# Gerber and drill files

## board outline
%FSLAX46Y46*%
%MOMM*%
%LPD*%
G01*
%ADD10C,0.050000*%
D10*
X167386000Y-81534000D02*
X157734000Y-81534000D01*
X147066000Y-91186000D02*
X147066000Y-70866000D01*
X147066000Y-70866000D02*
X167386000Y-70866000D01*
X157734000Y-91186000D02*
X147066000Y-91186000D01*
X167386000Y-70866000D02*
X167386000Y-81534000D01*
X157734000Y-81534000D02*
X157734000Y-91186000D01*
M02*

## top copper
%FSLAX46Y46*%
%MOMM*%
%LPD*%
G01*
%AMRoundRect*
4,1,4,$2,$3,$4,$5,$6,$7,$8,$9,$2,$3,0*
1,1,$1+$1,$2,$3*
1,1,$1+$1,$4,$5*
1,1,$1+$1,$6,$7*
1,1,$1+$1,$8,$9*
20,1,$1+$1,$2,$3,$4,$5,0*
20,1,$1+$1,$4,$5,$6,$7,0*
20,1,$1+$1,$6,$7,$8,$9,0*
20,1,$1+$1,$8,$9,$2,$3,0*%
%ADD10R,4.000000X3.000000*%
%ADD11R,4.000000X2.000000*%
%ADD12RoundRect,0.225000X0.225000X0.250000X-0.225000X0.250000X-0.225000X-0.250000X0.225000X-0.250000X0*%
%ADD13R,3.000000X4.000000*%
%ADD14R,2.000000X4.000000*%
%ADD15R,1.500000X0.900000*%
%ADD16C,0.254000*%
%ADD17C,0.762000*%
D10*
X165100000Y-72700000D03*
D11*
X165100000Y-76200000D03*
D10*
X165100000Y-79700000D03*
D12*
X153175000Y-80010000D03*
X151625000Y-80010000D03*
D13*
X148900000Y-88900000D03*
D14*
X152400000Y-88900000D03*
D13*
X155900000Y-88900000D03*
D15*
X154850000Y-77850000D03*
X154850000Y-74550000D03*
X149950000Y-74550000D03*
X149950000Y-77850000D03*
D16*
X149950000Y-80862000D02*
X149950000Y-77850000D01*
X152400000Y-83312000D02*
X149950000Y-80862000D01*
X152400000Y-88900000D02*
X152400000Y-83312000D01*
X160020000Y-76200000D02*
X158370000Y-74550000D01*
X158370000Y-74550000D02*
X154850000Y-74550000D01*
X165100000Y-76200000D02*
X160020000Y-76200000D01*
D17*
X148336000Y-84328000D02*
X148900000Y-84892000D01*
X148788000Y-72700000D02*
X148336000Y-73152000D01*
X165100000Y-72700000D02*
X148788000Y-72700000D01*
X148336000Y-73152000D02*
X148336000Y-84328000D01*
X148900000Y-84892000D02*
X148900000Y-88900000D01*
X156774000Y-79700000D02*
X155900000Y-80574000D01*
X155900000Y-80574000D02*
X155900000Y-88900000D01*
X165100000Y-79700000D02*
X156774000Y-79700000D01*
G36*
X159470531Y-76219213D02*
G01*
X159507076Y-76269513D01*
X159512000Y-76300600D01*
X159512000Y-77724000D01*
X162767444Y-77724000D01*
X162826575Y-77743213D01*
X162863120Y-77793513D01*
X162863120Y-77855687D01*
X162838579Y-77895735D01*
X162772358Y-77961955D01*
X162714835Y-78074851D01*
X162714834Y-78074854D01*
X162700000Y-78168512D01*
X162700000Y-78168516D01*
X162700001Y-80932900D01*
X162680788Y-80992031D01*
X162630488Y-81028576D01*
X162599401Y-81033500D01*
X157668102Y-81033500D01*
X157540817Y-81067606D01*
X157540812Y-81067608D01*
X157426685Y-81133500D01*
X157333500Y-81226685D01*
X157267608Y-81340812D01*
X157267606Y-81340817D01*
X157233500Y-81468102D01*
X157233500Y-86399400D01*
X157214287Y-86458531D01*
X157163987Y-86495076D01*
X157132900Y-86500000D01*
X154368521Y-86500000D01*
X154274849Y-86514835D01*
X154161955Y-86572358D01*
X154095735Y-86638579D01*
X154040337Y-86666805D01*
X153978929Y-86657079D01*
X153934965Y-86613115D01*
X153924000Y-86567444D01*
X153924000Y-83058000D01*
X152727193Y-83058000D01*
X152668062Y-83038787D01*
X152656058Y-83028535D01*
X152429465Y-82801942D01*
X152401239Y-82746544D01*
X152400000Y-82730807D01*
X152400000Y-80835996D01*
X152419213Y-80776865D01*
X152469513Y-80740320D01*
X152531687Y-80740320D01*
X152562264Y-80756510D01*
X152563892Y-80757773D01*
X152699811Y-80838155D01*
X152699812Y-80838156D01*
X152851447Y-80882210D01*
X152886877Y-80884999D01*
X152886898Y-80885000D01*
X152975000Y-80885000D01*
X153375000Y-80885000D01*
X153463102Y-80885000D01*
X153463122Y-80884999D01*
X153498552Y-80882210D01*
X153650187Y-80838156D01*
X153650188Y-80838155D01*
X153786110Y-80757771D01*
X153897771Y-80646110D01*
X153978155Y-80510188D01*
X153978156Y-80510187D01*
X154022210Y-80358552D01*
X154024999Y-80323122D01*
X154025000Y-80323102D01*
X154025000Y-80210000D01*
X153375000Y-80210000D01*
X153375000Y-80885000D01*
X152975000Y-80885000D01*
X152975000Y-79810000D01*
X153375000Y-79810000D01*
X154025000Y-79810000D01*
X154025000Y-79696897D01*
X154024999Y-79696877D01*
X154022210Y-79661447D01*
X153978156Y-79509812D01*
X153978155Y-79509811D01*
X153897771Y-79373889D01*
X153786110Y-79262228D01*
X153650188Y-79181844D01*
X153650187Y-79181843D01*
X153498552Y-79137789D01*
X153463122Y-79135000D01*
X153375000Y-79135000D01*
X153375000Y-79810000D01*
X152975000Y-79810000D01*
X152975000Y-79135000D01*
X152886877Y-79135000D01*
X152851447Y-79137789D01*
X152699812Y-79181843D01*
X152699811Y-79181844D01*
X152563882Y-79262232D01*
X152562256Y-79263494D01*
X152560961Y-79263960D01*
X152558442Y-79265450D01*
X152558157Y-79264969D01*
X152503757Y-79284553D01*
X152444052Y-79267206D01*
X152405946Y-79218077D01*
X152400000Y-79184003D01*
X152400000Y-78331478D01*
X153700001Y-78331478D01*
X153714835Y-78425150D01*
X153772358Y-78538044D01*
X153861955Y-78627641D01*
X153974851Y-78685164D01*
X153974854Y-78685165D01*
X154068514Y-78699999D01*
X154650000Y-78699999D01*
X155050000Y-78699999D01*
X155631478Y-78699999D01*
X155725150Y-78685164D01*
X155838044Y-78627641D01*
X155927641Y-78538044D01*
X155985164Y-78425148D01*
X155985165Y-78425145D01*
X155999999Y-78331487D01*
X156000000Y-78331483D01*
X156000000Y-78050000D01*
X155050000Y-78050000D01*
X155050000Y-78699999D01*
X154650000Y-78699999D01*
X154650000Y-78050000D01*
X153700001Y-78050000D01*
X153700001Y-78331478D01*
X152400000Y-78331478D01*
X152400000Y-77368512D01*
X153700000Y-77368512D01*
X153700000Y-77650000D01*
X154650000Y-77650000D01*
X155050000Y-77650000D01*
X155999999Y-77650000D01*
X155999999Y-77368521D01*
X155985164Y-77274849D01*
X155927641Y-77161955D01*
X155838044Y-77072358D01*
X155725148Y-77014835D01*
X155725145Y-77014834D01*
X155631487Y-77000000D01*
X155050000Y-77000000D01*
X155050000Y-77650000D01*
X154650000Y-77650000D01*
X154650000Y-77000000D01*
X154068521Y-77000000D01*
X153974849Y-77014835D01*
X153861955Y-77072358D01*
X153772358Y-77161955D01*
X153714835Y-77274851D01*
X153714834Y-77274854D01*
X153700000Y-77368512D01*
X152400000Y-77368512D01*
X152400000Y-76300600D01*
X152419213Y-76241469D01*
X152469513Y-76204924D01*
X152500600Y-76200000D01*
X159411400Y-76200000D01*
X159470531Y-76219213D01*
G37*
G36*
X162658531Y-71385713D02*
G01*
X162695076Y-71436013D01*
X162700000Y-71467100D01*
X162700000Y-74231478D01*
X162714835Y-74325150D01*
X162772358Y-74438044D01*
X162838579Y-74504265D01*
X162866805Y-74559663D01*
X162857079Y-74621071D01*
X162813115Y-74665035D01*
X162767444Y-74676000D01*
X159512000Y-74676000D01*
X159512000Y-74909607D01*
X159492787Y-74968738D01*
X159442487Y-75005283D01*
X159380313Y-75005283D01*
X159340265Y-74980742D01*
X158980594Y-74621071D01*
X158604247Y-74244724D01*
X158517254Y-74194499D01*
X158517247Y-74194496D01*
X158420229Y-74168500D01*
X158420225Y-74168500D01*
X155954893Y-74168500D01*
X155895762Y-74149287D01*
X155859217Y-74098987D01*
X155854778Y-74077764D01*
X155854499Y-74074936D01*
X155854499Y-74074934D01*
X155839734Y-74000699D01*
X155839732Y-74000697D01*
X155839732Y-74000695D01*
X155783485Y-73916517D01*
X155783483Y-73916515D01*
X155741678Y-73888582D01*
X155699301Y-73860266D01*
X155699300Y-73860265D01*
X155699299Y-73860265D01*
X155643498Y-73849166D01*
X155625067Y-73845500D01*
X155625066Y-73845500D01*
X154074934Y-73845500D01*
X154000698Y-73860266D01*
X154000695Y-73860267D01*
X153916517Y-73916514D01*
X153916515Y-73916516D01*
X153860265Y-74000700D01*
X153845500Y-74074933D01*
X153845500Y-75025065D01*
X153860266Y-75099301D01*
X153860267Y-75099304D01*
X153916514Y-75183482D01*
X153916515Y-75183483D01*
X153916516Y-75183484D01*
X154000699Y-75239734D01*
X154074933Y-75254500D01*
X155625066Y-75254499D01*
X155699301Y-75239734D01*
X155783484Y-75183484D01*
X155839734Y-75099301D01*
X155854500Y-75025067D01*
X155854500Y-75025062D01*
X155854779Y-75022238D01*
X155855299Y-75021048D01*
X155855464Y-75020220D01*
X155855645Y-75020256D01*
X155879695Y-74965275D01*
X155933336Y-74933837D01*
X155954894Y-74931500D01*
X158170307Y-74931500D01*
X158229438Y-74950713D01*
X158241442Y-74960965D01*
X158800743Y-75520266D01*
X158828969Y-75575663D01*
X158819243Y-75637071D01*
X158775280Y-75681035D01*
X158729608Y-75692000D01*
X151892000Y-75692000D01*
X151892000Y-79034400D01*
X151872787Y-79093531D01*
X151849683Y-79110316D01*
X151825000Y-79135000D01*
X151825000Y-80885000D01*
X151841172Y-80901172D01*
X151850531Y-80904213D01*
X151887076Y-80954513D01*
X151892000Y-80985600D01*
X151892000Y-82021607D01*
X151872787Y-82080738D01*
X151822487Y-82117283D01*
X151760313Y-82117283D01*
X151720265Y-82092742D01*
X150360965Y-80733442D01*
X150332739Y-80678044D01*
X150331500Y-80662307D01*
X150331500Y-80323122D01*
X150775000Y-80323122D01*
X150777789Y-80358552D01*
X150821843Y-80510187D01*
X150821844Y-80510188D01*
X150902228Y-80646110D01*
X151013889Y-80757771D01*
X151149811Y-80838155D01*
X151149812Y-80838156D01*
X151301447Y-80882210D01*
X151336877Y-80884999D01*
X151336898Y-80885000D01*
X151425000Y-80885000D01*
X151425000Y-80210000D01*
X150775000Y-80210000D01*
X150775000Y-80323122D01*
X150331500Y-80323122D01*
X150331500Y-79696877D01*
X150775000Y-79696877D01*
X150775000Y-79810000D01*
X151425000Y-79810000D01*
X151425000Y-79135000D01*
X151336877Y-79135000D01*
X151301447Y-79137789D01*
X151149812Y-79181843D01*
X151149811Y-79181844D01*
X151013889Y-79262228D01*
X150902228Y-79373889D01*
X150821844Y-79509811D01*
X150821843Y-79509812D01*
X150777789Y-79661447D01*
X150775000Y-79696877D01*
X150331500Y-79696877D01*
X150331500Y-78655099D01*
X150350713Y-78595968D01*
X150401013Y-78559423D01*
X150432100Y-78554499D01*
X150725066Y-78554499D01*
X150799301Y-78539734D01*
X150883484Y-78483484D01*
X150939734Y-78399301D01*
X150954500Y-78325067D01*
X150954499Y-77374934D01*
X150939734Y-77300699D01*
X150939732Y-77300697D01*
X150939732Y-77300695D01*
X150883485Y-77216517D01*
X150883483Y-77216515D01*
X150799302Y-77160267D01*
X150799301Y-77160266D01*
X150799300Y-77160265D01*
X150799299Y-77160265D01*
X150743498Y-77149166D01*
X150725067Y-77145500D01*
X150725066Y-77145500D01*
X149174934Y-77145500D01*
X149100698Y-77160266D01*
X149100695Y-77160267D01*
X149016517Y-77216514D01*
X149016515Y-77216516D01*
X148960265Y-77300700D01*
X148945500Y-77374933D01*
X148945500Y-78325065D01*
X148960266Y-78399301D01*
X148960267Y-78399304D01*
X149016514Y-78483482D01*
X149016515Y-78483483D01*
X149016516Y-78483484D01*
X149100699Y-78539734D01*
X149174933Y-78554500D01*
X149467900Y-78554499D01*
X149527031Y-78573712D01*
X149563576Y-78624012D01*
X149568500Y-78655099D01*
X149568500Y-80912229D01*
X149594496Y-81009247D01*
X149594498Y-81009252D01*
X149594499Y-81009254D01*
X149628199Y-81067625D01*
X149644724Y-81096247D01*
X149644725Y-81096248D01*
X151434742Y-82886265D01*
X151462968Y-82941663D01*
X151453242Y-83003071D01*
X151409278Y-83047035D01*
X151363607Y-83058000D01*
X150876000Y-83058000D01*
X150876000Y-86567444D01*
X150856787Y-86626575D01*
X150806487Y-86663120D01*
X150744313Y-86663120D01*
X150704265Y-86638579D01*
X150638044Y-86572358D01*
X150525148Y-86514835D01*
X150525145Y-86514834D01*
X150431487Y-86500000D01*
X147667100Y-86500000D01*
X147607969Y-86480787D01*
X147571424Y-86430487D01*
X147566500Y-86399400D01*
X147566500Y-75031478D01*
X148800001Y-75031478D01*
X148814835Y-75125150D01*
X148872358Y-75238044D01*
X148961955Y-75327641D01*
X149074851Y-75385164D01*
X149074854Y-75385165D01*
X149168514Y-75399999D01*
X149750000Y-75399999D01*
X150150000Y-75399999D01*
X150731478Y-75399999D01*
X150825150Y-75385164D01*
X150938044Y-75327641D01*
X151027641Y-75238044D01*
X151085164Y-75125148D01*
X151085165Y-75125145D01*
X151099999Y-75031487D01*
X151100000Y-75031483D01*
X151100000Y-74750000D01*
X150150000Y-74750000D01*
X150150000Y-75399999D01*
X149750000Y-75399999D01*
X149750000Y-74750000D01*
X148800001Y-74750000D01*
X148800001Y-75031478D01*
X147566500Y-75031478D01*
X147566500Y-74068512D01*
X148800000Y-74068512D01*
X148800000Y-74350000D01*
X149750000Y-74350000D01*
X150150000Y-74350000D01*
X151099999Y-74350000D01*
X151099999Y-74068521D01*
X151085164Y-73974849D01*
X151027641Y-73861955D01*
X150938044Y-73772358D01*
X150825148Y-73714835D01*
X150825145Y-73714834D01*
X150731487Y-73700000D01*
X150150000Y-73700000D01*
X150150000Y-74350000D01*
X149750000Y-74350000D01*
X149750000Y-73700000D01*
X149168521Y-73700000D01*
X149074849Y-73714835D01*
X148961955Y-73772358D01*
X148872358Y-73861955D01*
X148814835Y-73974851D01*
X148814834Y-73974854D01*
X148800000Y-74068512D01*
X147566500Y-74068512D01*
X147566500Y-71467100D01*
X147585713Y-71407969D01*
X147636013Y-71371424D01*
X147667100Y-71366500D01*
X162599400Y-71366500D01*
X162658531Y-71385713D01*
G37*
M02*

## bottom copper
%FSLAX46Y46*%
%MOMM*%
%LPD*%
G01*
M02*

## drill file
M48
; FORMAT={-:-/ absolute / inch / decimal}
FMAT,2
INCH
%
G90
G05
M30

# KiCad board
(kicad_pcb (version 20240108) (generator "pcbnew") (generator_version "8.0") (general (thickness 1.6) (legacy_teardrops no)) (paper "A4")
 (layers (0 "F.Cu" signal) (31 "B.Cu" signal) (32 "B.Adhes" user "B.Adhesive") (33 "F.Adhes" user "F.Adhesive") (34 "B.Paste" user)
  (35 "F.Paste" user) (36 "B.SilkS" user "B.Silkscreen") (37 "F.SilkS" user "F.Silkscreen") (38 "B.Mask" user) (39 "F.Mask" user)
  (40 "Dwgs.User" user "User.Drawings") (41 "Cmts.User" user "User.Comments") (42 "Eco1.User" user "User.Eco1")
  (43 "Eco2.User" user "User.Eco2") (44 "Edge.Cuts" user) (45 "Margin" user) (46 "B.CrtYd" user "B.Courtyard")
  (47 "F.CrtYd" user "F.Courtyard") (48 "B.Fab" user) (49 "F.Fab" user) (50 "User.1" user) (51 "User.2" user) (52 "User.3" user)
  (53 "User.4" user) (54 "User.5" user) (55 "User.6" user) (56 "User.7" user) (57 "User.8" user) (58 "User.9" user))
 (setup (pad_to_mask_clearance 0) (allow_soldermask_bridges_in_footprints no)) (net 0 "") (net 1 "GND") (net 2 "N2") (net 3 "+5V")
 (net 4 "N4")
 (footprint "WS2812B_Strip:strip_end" (layer "F.Cu") (at 165.1 76.2)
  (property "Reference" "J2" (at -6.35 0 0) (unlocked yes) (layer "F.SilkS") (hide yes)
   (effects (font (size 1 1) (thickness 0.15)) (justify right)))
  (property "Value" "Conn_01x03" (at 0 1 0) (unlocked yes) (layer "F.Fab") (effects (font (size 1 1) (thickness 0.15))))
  (pad "1" smd rect (at 0 -3.5) (size 4 3) (layers "F.Cu" "F.Paste" "F.Mask") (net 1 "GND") (thermal_bridge_angle 45))
  (pad "2" smd rect (at 0 0) (size 4 2) (layers "F.Cu" "F.Paste" "F.Mask") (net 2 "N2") (thermal_bridge_angle 45))
  (pad "3" smd rect (at 0 3.5) (size 4 3) (layers "F.Cu" "F.Paste" "F.Mask") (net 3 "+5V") (thermal_bridge_angle 45)))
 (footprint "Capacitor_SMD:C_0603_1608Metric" (layer "F.Cu") (at 152.4 80.01 180)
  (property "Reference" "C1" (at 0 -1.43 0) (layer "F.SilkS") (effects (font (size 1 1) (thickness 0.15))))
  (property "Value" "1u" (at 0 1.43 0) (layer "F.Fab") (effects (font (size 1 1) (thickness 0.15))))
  (pad "1" smd roundrect (at -0.775 0 180) (size 0.9 0.95) (layers "F.Cu" "F.Paste" "F.Mask") (roundrect_rratio 0.25) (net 3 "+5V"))
  (pad "2" smd roundrect (at 0.775 0 180) (size 0.9 0.95) (layers "F.Cu" "F.Paste" "F.Mask") (roundrect_rratio 0.25) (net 1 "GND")))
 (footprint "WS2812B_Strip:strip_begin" (layer "F.Cu") (at 152.4 88.9 90)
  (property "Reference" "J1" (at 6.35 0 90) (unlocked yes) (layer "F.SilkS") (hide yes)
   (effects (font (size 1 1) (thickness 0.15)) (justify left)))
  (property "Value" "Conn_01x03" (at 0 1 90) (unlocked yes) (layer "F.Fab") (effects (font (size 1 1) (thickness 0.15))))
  (pad "1" smd rect (at 0 -3.5 90) (size 4 3) (layers "F.Cu" "F.Paste" "F.Mask") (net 1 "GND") (thermal_bridge_angle 45))
  (pad "2" smd rect (at 0 0 90) (size 4 2) (layers "F.Cu" "F.Paste" "F.Mask") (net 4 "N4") (thermal_bridge_angle 45))
  (pad "3" smd rect (at 0 3.5 90) (size 4 3) (layers "F.Cu" "F.Paste" "F.Mask") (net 3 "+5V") (thermal_bridge_angle 45)))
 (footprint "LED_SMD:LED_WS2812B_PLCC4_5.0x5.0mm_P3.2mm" (layer "F.Cu") (at 152.4 76.2 180)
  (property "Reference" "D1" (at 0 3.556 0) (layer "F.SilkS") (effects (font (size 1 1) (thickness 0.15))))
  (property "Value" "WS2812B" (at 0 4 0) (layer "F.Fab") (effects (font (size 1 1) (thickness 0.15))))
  (pad "1" smd rect (at -2.45 -1.65 180) (size 1.5 0.9) (layers "F.Cu" "F.Paste" "F.Mask") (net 3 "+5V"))
  (pad "2" smd rect (at -2.45 1.65 180) (size 1.5 0.9) (layers "F.Cu" "F.Paste" "F.Mask") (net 2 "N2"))
  (pad "3" smd rect (at 2.45 1.65 180) (size 1.5 0.9) (layers "F.Cu" "F.Paste" "F.Mask") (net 1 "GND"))
  (pad "4" smd rect (at 2.45 -1.65 180) (size 1.5 0.9) (layers "F.Cu" "F.Paste" "F.Mask") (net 4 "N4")))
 (gr_line (start 167.386 81.534) (end 157.734 81.534) (stroke (width 0.05) (type default)) (layer "Edge.Cuts"))
 (gr_line (start 147.066 91.186) (end 147.066 70.866) (stroke (width 0.05) (type default)) (layer "Edge.Cuts"))
 (gr_line (start 147.066 70.866) (end 167.386 70.866) (stroke (width 0.05) (type default)) (layer "Edge.Cuts"))
 (gr_line (start 157.734 91.186) (end 147.066 91.186) (stroke (width 0.05) (type default)) (layer "Edge.Cuts"))
 (gr_line (start 167.386 70.866) (end 167.386 81.534) (stroke (width 0.05) (type default)) (layer "Edge.Cuts"))
 (gr_line (start 157.734 81.534) (end 157.734 91.186) (stroke (width 0.05) (type default)) (layer "Edge.Cuts"))
 (segment (start 149.95 80.862) (end 149.95 77.85) (width 0.254) (layer "F.Cu") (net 4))
 (segment (start 152.4 83.312) (end 149.95 80.862) (width 0.254) (layer "F.Cu") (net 4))
 (segment (start 152.4 88.9) (end 152.4 83.312) (width 0.254) (layer "F.Cu") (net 4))
 (segment (start 160.02 76.2) (end 158.37 74.55) (width 0.254) (layer "F.Cu") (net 2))
 (segment (start 158.37 74.55) (end 154.85 74.55) (width 0.254) (layer "F.Cu") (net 2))
 (segment (start 165.1 76.2) (end 160.02 76.2) (width 0.254) (layer "F.Cu") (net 2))
 (segment (start 148.336 84.328) (end 148.9 84.892) (width 0.762) (layer "F.Cu") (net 1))
 (segment (start 148.788 72.7) (end 148.336 73.152) (width 0.762) (layer "F.Cu") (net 1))
 (segment (start 165.1 72.7) (end 148.788 72.7) (width 0.762) (layer "F.Cu") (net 1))
 (segment (start 148.336 73.152) (end 148.336 84.328) (width 0.762) (layer "F.Cu") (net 1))
 (segment (start 148.9 84.892) (end 148.9 88.9) (width 0.762) (layer "F.Cu") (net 1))
 (segment (start 156.774 79.7) (end 155.9 80.574) (width 0.762) (layer "F.Cu") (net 3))
 (segment (start 155.9 80.574) (end 155.9 88.9) (width 0.762) (layer "F.Cu") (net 3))
 (segment (start 165.1 79.7) (end 156.774 79.7) (width 0.762) (layer "F.Cu") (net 3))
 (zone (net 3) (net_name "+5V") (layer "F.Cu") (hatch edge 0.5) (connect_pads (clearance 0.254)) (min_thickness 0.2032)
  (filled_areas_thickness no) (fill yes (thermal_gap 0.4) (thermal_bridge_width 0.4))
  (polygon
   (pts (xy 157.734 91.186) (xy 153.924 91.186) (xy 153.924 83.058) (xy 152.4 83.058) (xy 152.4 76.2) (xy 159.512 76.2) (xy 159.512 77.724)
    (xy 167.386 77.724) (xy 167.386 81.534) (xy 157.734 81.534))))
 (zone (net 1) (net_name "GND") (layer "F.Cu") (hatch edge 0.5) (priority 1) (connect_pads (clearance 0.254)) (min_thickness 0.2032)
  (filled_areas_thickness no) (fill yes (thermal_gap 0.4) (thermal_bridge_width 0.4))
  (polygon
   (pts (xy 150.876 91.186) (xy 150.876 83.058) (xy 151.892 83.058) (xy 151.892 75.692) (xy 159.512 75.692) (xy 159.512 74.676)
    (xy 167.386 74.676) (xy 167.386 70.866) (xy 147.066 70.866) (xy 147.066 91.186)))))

